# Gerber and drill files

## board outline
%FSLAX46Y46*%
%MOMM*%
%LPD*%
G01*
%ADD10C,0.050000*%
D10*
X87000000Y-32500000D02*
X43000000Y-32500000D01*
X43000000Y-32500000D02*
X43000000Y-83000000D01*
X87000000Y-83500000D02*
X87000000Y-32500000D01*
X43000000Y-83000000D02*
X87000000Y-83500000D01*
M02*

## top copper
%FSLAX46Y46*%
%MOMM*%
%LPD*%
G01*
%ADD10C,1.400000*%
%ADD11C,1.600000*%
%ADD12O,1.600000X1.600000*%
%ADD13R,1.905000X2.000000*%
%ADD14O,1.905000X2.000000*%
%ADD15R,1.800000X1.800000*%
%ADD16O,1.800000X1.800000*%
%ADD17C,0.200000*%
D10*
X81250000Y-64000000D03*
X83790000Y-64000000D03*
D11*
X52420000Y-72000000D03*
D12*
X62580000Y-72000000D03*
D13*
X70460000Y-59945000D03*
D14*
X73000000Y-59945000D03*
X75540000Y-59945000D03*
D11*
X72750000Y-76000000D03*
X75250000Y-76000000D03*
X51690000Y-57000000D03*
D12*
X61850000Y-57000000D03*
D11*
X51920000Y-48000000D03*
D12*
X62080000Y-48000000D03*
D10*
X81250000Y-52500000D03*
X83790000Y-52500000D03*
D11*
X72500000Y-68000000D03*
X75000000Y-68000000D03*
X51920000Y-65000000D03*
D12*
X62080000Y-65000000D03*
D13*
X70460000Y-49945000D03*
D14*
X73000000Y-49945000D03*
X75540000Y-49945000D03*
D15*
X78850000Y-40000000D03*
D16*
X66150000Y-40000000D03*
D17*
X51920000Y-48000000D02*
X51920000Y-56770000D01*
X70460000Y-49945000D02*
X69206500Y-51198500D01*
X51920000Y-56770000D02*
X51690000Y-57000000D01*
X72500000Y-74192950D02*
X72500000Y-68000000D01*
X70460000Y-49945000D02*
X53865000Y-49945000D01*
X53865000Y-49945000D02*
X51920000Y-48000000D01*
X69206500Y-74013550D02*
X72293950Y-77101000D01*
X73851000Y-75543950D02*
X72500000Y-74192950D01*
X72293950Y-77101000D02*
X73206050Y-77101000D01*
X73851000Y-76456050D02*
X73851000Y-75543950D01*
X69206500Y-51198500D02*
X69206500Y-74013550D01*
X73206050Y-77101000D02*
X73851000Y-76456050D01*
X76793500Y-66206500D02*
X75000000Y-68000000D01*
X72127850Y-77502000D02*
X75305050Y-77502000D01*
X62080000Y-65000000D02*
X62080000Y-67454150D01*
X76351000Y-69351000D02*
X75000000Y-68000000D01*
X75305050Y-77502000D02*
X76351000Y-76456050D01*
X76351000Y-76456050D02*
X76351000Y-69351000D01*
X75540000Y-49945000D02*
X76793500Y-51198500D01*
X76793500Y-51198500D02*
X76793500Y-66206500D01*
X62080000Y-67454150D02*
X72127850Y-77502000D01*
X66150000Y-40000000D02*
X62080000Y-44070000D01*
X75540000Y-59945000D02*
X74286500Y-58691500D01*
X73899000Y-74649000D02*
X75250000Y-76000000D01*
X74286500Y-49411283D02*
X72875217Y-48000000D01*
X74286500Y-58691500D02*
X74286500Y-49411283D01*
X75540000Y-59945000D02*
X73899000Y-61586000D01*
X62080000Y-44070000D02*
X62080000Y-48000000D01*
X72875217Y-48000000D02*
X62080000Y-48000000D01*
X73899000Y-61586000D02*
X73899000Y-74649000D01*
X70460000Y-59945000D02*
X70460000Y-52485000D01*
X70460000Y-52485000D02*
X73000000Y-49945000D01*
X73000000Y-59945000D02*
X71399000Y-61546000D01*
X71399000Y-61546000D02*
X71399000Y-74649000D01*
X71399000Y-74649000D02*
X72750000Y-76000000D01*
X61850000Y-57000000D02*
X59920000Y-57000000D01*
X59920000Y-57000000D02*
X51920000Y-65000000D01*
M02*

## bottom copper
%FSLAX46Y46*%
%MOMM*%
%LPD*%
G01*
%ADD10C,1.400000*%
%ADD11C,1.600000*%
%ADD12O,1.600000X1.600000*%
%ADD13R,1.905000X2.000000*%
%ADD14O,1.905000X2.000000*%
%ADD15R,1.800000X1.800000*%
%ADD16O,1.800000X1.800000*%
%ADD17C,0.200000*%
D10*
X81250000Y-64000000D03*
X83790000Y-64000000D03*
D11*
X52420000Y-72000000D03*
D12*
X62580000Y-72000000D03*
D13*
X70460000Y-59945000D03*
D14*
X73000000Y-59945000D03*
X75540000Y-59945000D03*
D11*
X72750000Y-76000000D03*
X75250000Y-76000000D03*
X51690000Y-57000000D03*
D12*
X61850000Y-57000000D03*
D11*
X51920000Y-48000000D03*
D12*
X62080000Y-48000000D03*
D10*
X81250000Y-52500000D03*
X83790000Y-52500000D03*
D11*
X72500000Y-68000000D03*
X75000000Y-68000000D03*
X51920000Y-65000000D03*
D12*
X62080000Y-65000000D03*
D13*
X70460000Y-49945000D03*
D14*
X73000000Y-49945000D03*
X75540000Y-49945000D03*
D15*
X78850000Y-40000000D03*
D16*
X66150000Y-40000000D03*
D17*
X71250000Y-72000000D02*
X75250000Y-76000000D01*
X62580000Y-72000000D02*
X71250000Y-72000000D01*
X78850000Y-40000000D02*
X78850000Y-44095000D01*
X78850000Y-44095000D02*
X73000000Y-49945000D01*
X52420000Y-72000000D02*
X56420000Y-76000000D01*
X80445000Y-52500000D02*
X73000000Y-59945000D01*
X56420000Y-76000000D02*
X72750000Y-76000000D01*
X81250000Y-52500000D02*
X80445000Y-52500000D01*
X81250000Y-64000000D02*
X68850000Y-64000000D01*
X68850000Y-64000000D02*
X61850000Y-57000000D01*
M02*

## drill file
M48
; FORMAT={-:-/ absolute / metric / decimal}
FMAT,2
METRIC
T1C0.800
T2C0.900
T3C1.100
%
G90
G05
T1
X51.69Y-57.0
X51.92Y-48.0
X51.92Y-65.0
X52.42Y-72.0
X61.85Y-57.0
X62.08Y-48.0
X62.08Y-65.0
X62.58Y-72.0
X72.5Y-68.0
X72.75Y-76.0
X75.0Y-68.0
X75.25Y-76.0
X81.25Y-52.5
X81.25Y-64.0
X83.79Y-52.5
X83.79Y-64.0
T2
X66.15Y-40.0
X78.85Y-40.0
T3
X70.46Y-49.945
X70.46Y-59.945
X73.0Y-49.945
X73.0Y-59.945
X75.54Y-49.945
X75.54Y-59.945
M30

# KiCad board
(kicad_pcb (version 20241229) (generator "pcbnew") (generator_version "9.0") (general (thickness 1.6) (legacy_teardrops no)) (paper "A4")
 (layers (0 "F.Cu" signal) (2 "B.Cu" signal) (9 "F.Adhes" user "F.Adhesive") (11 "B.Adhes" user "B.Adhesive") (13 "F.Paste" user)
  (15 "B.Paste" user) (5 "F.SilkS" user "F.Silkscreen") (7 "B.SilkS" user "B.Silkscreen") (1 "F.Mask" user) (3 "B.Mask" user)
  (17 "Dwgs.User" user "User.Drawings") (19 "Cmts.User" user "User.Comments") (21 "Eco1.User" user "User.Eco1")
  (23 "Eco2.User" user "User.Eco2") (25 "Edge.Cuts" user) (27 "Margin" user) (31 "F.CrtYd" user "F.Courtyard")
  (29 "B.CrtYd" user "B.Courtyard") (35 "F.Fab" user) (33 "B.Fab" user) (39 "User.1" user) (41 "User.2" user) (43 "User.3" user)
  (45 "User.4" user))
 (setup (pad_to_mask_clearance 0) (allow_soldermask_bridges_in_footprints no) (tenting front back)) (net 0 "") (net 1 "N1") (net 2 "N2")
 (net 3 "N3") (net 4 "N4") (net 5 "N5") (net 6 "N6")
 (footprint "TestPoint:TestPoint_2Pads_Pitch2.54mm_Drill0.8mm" (layer "F.Cu") (at 81.25 64)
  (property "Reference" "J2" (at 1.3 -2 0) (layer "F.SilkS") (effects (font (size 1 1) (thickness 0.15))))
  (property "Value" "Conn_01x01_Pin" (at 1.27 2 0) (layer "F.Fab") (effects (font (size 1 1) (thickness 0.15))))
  (pad "1" thru_hole circle (at 0 0) (size 1.4 1.4) (drill 0.8) (layers "*.Cu" "*.Mask") (remove_unused_layers no) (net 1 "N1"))
  (pad "2" thru_hole circle (at 2.54 0) (size 1.4 1.4) (drill 0.8) (layers "*.Cu" "*.Mask") (remove_unused_layers no)))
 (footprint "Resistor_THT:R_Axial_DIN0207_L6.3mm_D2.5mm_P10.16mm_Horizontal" (layer "F.Cu") (at 52.42 72)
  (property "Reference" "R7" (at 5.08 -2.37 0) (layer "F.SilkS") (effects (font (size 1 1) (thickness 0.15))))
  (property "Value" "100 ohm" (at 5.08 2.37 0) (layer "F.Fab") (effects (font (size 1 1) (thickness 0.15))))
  (pad "1" thru_hole circle (at 0 0) (size 1.6 1.6) (drill 0.8) (layers "*.Cu" "*.Mask") (remove_unused_layers no) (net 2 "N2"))
  (pad "2" thru_hole oval (at 10.16 0) (size 1.6 1.6) (drill 0.8) (layers "*.Cu" "*.Mask") (remove_unused_layers no) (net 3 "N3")))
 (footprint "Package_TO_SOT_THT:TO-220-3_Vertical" (layer "F.Cu") (at 70.46 59.945)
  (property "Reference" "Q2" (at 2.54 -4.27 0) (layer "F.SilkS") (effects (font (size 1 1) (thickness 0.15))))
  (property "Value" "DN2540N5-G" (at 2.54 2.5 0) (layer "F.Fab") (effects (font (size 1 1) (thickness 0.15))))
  (pad "1" thru_hole rect (at 0 0) (size 1.905 2) (drill 1.1) (layers "*.Cu" "*.Mask") (remove_unused_layers no) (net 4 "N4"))
  (pad "2" thru_hole oval (at 2.54 0) (size 1.905 2) (drill 1.1) (layers "*.Cu" "*.Mask") (remove_unused_layers no) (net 2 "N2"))
  (pad "3" thru_hole oval (at 5.08 0) (size 1.905 2) (drill 1.1) (layers "*.Cu" "*.Mask") (remove_unused_layers no) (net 3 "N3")))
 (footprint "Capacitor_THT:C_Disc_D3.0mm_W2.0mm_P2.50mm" (layer "F.Cu") (at 72.75 76)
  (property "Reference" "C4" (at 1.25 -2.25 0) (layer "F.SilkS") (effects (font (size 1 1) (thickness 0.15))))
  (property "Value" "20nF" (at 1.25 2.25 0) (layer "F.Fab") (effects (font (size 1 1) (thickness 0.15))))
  (pad "1" thru_hole circle (at 0 0) (size 1.6 1.6) (drill 0.8) (layers "*.Cu" "*.Mask") (remove_unused_layers no) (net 2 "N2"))
  (pad "2" thru_hole circle (at 2.5 0) (size 1.6 1.6) (drill 0.8) (layers "*.Cu" "*.Mask") (remove_unused_layers no) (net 3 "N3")))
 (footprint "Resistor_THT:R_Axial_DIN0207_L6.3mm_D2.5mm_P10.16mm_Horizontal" (layer "F.Cu") (at 51.69 57)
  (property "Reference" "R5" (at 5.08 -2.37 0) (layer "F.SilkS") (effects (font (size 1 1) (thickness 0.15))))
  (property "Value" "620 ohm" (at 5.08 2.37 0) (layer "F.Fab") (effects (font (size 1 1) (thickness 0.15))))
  (pad "1" thru_hole circle (at 0 0) (size 1.6 1.6) (drill 0.8) (layers "*.Cu" "*.Mask") (remove_unused_layers no) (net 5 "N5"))
  (pad "2" thru_hole oval (at 10.16 0) (size 1.6 1.6) (drill 0.8) (layers "*.Cu" "*.Mask") (remove_unused_layers no) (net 1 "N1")))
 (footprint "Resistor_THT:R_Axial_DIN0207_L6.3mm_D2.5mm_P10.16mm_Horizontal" (layer "F.Cu") (at 51.92 48)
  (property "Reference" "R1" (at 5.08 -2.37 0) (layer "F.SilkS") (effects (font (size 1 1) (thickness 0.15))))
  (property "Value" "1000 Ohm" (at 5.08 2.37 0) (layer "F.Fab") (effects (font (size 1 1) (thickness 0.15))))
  (pad "1" thru_hole circle (at 0 0) (size 1.6 1.6) (drill 0.8) (layers "*.Cu" "*.Mask") (remove_unused_layers no) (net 5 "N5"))
  (pad "2" thru_hole oval (at 10.16 0) (size 1.6 1.6) (drill 0.8) (layers "*.Cu" "*.Mask") (remove_unused_layers no) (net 3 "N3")))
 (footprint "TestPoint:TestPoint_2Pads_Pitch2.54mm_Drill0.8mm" (layer "F.Cu") (at 81.25 52.5)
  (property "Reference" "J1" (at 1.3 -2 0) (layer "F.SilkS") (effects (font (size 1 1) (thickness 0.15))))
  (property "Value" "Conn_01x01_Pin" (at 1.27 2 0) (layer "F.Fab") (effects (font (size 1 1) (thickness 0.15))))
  (pad "1" thru_hole circle (at 0 0) (size 1.4 1.4) (drill 0.8) (layers "*.Cu" "*.Mask") (remove_unused_layers no) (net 2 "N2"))
  (pad "2" thru_hole circle (at 2.54 0) (size 1.4 1.4) (drill 0.8) (layers "*.Cu" "*.Mask") (remove_unused_layers no)))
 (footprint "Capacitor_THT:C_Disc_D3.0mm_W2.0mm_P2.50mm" (layer "F.Cu") (at 72.5 68)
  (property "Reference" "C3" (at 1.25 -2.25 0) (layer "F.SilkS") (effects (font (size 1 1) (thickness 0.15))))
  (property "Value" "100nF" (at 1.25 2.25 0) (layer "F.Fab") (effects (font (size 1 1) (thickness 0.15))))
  (pad "1" thru_hole circle (at 0 0) (size 1.6 1.6) (drill 0.8) (layers "*.Cu" "*.Mask") (remove_unused_layers no) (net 5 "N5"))
  (pad "2" thru_hole circle (at 2.5 0) (size 1.6 1.6) (drill 0.8) (layers "*.Cu" "*.Mask") (remove_unused_layers no) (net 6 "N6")))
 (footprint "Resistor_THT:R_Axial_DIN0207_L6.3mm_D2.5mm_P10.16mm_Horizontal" (layer "F.Cu") (at 51.92 65)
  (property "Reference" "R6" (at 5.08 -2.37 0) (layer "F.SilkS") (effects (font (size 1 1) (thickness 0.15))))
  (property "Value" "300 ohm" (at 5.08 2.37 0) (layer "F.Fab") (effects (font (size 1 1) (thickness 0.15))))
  (pad "1" thru_hole circle (at 0 0) (size 1.6 1.6) (drill 0.8) (layers "*.Cu" "*.Mask") (remove_unused_layers no) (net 1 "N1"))
  (pad "2" thru_hole oval (at 10.16 0) (size 1.6 1.6) (drill 0.8) (layers "*.Cu" "*.Mask") (remove_unused_layers no) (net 6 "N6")))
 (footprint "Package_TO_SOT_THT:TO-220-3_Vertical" (layer "F.Cu") (at 70.46 49.945)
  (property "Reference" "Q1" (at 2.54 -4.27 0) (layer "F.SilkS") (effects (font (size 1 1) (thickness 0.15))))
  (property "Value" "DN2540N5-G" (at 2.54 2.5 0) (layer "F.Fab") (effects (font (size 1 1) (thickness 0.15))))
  (pad "1" thru_hole rect (at 0 0) (size 1.905 2) (drill 1.1) (layers "*.Cu" "*.Mask") (remove_unused_layers no) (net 5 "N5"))
  (pad "2" thru_hole oval (at 2.54 0) (size 1.905 2) (drill 1.1) (layers "*.Cu" "*.Mask") (remove_unused_layers no) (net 4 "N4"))
  (pad "3" thru_hole oval (at 5.08 0) (size 1.905 2) (drill 1.1) (layers "*.Cu" "*.Mask") (remove_unused_layers no) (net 6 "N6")))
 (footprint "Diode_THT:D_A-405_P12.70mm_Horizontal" (layer "F.Cu") (at 78.85 40 180)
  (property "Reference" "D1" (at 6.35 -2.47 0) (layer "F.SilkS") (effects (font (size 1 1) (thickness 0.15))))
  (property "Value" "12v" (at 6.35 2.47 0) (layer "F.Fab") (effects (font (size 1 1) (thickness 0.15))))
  (pad "1" thru_hole rect (at 0 0 180) (size 1.8 1.8) (drill 0.9) (layers "*.Cu" "*.Mask") (remove_unused_layers no) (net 4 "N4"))
  (pad "2" thru_hole oval (at 12.7 0 180) (size 1.8 1.8) (drill 0.9) (layers "*.Cu" "*.Mask") (remove_unused_layers no) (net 3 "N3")))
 (gr_line (start 87 32.5) (end 43 32.5) (stroke (width 0.05) (type default)) (layer "Edge.Cuts"))
 (gr_line (start 43 32.5) (end 43 83) (stroke (width 0.05) (type default)) (layer "Edge.Cuts"))
 (gr_line (start 87 83.5) (end 87 32.5) (stroke (width 0.05) (type default)) (layer "Edge.Cuts"))
 (gr_line (start 43 83) (end 87 83.5) (stroke (width 0.05) (type default)) (layer "Edge.Cuts"))
 (segment (start 51.92 48) (end 51.92 56.77) (width 0.2) (layer "F.Cu") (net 5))
 (segment (start 70.46 49.945) (end 69.2065 51.1985) (width 0.2) (layer "F.Cu") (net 5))
 (segment (start 51.92 56.77) (end 51.69 57) (width 0.2) (layer "F.Cu") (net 5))
 (segment (start 72.5 74.19295) (end 72.5 68) (width 0.2) (layer "F.Cu") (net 5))
 (segment (start 70.46 49.945) (end 53.865 49.945) (width 0.2) (layer "F.Cu") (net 5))
 (segment (start 53.865 49.945) (end 51.92 48) (width 0.2) (layer "F.Cu") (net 5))
 (segment (start 69.2065 74.01355) (end 72.29395 77.101) (width 0.2) (layer "F.Cu") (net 5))
 (segment (start 73.851 75.54395) (end 72.5 74.19295) (width 0.2) (layer "F.Cu") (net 5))
 (segment (start 72.29395 77.101) (end 73.20605 77.101) (width 0.2) (layer "F.Cu") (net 5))
 (segment (start 73.851 76.45605) (end 73.851 75.54395) (width 0.2) (layer "F.Cu") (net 5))
 (segment (start 69.2065 51.1985) (end 69.2065 74.01355) (width 0.2) (layer "F.Cu") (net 5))
 (segment (start 73.20605 77.101) (end 73.851 76.45605) (width 0.2) (layer "F.Cu") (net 5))
 (segment (start 76.7935 66.2065) (end 75 68) (width 0.2) (layer "F.Cu") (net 6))
 (segment (start 72.12785 77.502) (end 75.30505 77.502) (width 0.2) (layer "F.Cu") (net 6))
 (segment (start 62.08 65) (end 62.08 67.45415) (width 0.2) (layer "F.Cu") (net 6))
 (segment (start 76.351 69.351) (end 75 68) (width 0.2) (layer "F.Cu") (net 6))
 (segment (start 75.30505 77.502) (end 76.351 76.45605) (width 0.2) (layer "F.Cu") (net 6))
 (segment (start 76.351 76.45605) (end 76.351 69.351) (width 0.2) (layer "F.Cu") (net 6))
 (segment (start 75.54 49.945) (end 76.7935 51.1985) (width 0.2) (layer "F.Cu") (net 6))
 (segment (start 76.7935 51.1985) (end 76.7935 66.2065) (width 0.2) (layer "F.Cu") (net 6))
 (segment (start 62.08 67.45415) (end 72.12785 77.502) (width 0.2) (layer "F.Cu") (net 6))
 (segment (start 66.15 40) (end 62.08 44.07) (width 0.2) (layer "F.Cu") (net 3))
 (segment (start 75.54 59.945) (end 74.2865 58.6915) (width 0.2) (layer "F.Cu") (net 3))
 (segment (start 73.899 74.649) (end 75.25 76) (width 0.2) (layer "F.Cu") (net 3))
 (segment (start 74.2865 49.411283) (end 72.875217 48) (width 0.2) (layer "F.Cu") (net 3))
 (segment (start 74.2865 58.6915) (end 74.2865 49.411283) (width 0.2) (layer "F.Cu") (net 3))
 (segment (start 75.54 59.945) (end 73.899 61.586) (width 0.2) (layer "F.Cu") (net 3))
 (segment (start 62.08 44.07) (end 62.08 48) (width 0.2) (layer "F.Cu") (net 3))
 (segment (start 72.875217 48) (end 62.08 48) (width 0.2) (layer "F.Cu") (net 3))
 (segment (start 73.899 61.586) (end 73.899 74.649) (width 0.2) (layer "F.Cu") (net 3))
 (segment (start 71.25 72) (end 75.25 76) (width 0.2) (layer "B.Cu") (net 3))
 (segment (start 62.58 72) (end 71.25 72) (width 0.2) (layer "B.Cu") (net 3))
 (segment (start 70.46 59.945) (end 70.46 52.485) (width 0.2) (layer "F.Cu") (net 4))
 (segment (start 70.46 52.485) (end 73 49.945) (width 0.2) (layer "F.Cu") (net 4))
 (segment (start 78.85 40) (end 78.85 44.095) (width 0.2) (layer "B.Cu") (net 4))
 (segment (start 78.85 44.095) (end 73 49.945) (width 0.2) (layer "B.Cu") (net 4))
 (segment (start 73 59.945) (end 71.399 61.546) (width 0.2) (layer "F.Cu") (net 2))
 (segment (start 71.399 61.546) (end 71.399 74.649) (width 0.2) (layer "F.Cu") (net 2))
 (segment (start 71.399 74.649) (end 72.75 76) (width 0.2) (layer "F.Cu") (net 2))
 (segment (start 52.42 72) (end 56.42 76) (width 0.2) (layer "B.Cu") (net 2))
 (segment (start 80.445 52.5) (end 73 59.945) (width 0.2) (layer "B.Cu") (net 2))
 (segment (start 56.42 76) (end 72.75 76) (width 0.2) (layer "B.Cu") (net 2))
 (segment (start 81.25 52.5) (end 80.445 52.5) (width 0.2) (layer "B.Cu") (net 2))
 (segment (start 61.85 57) (end 59.92 57) (width 0.2) (layer "F.Cu") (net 1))
 (segment (start 59.92 57) (end 51.92 65) (width 0.2) (layer "F.Cu") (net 1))
 (segment (start 81.25 64) (end 68.85 64) (width 0.2) (layer "B.Cu") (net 1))
 (segment (start 68.85 64) (end 61.85 57) (width 0.2) (layer "B.Cu") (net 1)))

